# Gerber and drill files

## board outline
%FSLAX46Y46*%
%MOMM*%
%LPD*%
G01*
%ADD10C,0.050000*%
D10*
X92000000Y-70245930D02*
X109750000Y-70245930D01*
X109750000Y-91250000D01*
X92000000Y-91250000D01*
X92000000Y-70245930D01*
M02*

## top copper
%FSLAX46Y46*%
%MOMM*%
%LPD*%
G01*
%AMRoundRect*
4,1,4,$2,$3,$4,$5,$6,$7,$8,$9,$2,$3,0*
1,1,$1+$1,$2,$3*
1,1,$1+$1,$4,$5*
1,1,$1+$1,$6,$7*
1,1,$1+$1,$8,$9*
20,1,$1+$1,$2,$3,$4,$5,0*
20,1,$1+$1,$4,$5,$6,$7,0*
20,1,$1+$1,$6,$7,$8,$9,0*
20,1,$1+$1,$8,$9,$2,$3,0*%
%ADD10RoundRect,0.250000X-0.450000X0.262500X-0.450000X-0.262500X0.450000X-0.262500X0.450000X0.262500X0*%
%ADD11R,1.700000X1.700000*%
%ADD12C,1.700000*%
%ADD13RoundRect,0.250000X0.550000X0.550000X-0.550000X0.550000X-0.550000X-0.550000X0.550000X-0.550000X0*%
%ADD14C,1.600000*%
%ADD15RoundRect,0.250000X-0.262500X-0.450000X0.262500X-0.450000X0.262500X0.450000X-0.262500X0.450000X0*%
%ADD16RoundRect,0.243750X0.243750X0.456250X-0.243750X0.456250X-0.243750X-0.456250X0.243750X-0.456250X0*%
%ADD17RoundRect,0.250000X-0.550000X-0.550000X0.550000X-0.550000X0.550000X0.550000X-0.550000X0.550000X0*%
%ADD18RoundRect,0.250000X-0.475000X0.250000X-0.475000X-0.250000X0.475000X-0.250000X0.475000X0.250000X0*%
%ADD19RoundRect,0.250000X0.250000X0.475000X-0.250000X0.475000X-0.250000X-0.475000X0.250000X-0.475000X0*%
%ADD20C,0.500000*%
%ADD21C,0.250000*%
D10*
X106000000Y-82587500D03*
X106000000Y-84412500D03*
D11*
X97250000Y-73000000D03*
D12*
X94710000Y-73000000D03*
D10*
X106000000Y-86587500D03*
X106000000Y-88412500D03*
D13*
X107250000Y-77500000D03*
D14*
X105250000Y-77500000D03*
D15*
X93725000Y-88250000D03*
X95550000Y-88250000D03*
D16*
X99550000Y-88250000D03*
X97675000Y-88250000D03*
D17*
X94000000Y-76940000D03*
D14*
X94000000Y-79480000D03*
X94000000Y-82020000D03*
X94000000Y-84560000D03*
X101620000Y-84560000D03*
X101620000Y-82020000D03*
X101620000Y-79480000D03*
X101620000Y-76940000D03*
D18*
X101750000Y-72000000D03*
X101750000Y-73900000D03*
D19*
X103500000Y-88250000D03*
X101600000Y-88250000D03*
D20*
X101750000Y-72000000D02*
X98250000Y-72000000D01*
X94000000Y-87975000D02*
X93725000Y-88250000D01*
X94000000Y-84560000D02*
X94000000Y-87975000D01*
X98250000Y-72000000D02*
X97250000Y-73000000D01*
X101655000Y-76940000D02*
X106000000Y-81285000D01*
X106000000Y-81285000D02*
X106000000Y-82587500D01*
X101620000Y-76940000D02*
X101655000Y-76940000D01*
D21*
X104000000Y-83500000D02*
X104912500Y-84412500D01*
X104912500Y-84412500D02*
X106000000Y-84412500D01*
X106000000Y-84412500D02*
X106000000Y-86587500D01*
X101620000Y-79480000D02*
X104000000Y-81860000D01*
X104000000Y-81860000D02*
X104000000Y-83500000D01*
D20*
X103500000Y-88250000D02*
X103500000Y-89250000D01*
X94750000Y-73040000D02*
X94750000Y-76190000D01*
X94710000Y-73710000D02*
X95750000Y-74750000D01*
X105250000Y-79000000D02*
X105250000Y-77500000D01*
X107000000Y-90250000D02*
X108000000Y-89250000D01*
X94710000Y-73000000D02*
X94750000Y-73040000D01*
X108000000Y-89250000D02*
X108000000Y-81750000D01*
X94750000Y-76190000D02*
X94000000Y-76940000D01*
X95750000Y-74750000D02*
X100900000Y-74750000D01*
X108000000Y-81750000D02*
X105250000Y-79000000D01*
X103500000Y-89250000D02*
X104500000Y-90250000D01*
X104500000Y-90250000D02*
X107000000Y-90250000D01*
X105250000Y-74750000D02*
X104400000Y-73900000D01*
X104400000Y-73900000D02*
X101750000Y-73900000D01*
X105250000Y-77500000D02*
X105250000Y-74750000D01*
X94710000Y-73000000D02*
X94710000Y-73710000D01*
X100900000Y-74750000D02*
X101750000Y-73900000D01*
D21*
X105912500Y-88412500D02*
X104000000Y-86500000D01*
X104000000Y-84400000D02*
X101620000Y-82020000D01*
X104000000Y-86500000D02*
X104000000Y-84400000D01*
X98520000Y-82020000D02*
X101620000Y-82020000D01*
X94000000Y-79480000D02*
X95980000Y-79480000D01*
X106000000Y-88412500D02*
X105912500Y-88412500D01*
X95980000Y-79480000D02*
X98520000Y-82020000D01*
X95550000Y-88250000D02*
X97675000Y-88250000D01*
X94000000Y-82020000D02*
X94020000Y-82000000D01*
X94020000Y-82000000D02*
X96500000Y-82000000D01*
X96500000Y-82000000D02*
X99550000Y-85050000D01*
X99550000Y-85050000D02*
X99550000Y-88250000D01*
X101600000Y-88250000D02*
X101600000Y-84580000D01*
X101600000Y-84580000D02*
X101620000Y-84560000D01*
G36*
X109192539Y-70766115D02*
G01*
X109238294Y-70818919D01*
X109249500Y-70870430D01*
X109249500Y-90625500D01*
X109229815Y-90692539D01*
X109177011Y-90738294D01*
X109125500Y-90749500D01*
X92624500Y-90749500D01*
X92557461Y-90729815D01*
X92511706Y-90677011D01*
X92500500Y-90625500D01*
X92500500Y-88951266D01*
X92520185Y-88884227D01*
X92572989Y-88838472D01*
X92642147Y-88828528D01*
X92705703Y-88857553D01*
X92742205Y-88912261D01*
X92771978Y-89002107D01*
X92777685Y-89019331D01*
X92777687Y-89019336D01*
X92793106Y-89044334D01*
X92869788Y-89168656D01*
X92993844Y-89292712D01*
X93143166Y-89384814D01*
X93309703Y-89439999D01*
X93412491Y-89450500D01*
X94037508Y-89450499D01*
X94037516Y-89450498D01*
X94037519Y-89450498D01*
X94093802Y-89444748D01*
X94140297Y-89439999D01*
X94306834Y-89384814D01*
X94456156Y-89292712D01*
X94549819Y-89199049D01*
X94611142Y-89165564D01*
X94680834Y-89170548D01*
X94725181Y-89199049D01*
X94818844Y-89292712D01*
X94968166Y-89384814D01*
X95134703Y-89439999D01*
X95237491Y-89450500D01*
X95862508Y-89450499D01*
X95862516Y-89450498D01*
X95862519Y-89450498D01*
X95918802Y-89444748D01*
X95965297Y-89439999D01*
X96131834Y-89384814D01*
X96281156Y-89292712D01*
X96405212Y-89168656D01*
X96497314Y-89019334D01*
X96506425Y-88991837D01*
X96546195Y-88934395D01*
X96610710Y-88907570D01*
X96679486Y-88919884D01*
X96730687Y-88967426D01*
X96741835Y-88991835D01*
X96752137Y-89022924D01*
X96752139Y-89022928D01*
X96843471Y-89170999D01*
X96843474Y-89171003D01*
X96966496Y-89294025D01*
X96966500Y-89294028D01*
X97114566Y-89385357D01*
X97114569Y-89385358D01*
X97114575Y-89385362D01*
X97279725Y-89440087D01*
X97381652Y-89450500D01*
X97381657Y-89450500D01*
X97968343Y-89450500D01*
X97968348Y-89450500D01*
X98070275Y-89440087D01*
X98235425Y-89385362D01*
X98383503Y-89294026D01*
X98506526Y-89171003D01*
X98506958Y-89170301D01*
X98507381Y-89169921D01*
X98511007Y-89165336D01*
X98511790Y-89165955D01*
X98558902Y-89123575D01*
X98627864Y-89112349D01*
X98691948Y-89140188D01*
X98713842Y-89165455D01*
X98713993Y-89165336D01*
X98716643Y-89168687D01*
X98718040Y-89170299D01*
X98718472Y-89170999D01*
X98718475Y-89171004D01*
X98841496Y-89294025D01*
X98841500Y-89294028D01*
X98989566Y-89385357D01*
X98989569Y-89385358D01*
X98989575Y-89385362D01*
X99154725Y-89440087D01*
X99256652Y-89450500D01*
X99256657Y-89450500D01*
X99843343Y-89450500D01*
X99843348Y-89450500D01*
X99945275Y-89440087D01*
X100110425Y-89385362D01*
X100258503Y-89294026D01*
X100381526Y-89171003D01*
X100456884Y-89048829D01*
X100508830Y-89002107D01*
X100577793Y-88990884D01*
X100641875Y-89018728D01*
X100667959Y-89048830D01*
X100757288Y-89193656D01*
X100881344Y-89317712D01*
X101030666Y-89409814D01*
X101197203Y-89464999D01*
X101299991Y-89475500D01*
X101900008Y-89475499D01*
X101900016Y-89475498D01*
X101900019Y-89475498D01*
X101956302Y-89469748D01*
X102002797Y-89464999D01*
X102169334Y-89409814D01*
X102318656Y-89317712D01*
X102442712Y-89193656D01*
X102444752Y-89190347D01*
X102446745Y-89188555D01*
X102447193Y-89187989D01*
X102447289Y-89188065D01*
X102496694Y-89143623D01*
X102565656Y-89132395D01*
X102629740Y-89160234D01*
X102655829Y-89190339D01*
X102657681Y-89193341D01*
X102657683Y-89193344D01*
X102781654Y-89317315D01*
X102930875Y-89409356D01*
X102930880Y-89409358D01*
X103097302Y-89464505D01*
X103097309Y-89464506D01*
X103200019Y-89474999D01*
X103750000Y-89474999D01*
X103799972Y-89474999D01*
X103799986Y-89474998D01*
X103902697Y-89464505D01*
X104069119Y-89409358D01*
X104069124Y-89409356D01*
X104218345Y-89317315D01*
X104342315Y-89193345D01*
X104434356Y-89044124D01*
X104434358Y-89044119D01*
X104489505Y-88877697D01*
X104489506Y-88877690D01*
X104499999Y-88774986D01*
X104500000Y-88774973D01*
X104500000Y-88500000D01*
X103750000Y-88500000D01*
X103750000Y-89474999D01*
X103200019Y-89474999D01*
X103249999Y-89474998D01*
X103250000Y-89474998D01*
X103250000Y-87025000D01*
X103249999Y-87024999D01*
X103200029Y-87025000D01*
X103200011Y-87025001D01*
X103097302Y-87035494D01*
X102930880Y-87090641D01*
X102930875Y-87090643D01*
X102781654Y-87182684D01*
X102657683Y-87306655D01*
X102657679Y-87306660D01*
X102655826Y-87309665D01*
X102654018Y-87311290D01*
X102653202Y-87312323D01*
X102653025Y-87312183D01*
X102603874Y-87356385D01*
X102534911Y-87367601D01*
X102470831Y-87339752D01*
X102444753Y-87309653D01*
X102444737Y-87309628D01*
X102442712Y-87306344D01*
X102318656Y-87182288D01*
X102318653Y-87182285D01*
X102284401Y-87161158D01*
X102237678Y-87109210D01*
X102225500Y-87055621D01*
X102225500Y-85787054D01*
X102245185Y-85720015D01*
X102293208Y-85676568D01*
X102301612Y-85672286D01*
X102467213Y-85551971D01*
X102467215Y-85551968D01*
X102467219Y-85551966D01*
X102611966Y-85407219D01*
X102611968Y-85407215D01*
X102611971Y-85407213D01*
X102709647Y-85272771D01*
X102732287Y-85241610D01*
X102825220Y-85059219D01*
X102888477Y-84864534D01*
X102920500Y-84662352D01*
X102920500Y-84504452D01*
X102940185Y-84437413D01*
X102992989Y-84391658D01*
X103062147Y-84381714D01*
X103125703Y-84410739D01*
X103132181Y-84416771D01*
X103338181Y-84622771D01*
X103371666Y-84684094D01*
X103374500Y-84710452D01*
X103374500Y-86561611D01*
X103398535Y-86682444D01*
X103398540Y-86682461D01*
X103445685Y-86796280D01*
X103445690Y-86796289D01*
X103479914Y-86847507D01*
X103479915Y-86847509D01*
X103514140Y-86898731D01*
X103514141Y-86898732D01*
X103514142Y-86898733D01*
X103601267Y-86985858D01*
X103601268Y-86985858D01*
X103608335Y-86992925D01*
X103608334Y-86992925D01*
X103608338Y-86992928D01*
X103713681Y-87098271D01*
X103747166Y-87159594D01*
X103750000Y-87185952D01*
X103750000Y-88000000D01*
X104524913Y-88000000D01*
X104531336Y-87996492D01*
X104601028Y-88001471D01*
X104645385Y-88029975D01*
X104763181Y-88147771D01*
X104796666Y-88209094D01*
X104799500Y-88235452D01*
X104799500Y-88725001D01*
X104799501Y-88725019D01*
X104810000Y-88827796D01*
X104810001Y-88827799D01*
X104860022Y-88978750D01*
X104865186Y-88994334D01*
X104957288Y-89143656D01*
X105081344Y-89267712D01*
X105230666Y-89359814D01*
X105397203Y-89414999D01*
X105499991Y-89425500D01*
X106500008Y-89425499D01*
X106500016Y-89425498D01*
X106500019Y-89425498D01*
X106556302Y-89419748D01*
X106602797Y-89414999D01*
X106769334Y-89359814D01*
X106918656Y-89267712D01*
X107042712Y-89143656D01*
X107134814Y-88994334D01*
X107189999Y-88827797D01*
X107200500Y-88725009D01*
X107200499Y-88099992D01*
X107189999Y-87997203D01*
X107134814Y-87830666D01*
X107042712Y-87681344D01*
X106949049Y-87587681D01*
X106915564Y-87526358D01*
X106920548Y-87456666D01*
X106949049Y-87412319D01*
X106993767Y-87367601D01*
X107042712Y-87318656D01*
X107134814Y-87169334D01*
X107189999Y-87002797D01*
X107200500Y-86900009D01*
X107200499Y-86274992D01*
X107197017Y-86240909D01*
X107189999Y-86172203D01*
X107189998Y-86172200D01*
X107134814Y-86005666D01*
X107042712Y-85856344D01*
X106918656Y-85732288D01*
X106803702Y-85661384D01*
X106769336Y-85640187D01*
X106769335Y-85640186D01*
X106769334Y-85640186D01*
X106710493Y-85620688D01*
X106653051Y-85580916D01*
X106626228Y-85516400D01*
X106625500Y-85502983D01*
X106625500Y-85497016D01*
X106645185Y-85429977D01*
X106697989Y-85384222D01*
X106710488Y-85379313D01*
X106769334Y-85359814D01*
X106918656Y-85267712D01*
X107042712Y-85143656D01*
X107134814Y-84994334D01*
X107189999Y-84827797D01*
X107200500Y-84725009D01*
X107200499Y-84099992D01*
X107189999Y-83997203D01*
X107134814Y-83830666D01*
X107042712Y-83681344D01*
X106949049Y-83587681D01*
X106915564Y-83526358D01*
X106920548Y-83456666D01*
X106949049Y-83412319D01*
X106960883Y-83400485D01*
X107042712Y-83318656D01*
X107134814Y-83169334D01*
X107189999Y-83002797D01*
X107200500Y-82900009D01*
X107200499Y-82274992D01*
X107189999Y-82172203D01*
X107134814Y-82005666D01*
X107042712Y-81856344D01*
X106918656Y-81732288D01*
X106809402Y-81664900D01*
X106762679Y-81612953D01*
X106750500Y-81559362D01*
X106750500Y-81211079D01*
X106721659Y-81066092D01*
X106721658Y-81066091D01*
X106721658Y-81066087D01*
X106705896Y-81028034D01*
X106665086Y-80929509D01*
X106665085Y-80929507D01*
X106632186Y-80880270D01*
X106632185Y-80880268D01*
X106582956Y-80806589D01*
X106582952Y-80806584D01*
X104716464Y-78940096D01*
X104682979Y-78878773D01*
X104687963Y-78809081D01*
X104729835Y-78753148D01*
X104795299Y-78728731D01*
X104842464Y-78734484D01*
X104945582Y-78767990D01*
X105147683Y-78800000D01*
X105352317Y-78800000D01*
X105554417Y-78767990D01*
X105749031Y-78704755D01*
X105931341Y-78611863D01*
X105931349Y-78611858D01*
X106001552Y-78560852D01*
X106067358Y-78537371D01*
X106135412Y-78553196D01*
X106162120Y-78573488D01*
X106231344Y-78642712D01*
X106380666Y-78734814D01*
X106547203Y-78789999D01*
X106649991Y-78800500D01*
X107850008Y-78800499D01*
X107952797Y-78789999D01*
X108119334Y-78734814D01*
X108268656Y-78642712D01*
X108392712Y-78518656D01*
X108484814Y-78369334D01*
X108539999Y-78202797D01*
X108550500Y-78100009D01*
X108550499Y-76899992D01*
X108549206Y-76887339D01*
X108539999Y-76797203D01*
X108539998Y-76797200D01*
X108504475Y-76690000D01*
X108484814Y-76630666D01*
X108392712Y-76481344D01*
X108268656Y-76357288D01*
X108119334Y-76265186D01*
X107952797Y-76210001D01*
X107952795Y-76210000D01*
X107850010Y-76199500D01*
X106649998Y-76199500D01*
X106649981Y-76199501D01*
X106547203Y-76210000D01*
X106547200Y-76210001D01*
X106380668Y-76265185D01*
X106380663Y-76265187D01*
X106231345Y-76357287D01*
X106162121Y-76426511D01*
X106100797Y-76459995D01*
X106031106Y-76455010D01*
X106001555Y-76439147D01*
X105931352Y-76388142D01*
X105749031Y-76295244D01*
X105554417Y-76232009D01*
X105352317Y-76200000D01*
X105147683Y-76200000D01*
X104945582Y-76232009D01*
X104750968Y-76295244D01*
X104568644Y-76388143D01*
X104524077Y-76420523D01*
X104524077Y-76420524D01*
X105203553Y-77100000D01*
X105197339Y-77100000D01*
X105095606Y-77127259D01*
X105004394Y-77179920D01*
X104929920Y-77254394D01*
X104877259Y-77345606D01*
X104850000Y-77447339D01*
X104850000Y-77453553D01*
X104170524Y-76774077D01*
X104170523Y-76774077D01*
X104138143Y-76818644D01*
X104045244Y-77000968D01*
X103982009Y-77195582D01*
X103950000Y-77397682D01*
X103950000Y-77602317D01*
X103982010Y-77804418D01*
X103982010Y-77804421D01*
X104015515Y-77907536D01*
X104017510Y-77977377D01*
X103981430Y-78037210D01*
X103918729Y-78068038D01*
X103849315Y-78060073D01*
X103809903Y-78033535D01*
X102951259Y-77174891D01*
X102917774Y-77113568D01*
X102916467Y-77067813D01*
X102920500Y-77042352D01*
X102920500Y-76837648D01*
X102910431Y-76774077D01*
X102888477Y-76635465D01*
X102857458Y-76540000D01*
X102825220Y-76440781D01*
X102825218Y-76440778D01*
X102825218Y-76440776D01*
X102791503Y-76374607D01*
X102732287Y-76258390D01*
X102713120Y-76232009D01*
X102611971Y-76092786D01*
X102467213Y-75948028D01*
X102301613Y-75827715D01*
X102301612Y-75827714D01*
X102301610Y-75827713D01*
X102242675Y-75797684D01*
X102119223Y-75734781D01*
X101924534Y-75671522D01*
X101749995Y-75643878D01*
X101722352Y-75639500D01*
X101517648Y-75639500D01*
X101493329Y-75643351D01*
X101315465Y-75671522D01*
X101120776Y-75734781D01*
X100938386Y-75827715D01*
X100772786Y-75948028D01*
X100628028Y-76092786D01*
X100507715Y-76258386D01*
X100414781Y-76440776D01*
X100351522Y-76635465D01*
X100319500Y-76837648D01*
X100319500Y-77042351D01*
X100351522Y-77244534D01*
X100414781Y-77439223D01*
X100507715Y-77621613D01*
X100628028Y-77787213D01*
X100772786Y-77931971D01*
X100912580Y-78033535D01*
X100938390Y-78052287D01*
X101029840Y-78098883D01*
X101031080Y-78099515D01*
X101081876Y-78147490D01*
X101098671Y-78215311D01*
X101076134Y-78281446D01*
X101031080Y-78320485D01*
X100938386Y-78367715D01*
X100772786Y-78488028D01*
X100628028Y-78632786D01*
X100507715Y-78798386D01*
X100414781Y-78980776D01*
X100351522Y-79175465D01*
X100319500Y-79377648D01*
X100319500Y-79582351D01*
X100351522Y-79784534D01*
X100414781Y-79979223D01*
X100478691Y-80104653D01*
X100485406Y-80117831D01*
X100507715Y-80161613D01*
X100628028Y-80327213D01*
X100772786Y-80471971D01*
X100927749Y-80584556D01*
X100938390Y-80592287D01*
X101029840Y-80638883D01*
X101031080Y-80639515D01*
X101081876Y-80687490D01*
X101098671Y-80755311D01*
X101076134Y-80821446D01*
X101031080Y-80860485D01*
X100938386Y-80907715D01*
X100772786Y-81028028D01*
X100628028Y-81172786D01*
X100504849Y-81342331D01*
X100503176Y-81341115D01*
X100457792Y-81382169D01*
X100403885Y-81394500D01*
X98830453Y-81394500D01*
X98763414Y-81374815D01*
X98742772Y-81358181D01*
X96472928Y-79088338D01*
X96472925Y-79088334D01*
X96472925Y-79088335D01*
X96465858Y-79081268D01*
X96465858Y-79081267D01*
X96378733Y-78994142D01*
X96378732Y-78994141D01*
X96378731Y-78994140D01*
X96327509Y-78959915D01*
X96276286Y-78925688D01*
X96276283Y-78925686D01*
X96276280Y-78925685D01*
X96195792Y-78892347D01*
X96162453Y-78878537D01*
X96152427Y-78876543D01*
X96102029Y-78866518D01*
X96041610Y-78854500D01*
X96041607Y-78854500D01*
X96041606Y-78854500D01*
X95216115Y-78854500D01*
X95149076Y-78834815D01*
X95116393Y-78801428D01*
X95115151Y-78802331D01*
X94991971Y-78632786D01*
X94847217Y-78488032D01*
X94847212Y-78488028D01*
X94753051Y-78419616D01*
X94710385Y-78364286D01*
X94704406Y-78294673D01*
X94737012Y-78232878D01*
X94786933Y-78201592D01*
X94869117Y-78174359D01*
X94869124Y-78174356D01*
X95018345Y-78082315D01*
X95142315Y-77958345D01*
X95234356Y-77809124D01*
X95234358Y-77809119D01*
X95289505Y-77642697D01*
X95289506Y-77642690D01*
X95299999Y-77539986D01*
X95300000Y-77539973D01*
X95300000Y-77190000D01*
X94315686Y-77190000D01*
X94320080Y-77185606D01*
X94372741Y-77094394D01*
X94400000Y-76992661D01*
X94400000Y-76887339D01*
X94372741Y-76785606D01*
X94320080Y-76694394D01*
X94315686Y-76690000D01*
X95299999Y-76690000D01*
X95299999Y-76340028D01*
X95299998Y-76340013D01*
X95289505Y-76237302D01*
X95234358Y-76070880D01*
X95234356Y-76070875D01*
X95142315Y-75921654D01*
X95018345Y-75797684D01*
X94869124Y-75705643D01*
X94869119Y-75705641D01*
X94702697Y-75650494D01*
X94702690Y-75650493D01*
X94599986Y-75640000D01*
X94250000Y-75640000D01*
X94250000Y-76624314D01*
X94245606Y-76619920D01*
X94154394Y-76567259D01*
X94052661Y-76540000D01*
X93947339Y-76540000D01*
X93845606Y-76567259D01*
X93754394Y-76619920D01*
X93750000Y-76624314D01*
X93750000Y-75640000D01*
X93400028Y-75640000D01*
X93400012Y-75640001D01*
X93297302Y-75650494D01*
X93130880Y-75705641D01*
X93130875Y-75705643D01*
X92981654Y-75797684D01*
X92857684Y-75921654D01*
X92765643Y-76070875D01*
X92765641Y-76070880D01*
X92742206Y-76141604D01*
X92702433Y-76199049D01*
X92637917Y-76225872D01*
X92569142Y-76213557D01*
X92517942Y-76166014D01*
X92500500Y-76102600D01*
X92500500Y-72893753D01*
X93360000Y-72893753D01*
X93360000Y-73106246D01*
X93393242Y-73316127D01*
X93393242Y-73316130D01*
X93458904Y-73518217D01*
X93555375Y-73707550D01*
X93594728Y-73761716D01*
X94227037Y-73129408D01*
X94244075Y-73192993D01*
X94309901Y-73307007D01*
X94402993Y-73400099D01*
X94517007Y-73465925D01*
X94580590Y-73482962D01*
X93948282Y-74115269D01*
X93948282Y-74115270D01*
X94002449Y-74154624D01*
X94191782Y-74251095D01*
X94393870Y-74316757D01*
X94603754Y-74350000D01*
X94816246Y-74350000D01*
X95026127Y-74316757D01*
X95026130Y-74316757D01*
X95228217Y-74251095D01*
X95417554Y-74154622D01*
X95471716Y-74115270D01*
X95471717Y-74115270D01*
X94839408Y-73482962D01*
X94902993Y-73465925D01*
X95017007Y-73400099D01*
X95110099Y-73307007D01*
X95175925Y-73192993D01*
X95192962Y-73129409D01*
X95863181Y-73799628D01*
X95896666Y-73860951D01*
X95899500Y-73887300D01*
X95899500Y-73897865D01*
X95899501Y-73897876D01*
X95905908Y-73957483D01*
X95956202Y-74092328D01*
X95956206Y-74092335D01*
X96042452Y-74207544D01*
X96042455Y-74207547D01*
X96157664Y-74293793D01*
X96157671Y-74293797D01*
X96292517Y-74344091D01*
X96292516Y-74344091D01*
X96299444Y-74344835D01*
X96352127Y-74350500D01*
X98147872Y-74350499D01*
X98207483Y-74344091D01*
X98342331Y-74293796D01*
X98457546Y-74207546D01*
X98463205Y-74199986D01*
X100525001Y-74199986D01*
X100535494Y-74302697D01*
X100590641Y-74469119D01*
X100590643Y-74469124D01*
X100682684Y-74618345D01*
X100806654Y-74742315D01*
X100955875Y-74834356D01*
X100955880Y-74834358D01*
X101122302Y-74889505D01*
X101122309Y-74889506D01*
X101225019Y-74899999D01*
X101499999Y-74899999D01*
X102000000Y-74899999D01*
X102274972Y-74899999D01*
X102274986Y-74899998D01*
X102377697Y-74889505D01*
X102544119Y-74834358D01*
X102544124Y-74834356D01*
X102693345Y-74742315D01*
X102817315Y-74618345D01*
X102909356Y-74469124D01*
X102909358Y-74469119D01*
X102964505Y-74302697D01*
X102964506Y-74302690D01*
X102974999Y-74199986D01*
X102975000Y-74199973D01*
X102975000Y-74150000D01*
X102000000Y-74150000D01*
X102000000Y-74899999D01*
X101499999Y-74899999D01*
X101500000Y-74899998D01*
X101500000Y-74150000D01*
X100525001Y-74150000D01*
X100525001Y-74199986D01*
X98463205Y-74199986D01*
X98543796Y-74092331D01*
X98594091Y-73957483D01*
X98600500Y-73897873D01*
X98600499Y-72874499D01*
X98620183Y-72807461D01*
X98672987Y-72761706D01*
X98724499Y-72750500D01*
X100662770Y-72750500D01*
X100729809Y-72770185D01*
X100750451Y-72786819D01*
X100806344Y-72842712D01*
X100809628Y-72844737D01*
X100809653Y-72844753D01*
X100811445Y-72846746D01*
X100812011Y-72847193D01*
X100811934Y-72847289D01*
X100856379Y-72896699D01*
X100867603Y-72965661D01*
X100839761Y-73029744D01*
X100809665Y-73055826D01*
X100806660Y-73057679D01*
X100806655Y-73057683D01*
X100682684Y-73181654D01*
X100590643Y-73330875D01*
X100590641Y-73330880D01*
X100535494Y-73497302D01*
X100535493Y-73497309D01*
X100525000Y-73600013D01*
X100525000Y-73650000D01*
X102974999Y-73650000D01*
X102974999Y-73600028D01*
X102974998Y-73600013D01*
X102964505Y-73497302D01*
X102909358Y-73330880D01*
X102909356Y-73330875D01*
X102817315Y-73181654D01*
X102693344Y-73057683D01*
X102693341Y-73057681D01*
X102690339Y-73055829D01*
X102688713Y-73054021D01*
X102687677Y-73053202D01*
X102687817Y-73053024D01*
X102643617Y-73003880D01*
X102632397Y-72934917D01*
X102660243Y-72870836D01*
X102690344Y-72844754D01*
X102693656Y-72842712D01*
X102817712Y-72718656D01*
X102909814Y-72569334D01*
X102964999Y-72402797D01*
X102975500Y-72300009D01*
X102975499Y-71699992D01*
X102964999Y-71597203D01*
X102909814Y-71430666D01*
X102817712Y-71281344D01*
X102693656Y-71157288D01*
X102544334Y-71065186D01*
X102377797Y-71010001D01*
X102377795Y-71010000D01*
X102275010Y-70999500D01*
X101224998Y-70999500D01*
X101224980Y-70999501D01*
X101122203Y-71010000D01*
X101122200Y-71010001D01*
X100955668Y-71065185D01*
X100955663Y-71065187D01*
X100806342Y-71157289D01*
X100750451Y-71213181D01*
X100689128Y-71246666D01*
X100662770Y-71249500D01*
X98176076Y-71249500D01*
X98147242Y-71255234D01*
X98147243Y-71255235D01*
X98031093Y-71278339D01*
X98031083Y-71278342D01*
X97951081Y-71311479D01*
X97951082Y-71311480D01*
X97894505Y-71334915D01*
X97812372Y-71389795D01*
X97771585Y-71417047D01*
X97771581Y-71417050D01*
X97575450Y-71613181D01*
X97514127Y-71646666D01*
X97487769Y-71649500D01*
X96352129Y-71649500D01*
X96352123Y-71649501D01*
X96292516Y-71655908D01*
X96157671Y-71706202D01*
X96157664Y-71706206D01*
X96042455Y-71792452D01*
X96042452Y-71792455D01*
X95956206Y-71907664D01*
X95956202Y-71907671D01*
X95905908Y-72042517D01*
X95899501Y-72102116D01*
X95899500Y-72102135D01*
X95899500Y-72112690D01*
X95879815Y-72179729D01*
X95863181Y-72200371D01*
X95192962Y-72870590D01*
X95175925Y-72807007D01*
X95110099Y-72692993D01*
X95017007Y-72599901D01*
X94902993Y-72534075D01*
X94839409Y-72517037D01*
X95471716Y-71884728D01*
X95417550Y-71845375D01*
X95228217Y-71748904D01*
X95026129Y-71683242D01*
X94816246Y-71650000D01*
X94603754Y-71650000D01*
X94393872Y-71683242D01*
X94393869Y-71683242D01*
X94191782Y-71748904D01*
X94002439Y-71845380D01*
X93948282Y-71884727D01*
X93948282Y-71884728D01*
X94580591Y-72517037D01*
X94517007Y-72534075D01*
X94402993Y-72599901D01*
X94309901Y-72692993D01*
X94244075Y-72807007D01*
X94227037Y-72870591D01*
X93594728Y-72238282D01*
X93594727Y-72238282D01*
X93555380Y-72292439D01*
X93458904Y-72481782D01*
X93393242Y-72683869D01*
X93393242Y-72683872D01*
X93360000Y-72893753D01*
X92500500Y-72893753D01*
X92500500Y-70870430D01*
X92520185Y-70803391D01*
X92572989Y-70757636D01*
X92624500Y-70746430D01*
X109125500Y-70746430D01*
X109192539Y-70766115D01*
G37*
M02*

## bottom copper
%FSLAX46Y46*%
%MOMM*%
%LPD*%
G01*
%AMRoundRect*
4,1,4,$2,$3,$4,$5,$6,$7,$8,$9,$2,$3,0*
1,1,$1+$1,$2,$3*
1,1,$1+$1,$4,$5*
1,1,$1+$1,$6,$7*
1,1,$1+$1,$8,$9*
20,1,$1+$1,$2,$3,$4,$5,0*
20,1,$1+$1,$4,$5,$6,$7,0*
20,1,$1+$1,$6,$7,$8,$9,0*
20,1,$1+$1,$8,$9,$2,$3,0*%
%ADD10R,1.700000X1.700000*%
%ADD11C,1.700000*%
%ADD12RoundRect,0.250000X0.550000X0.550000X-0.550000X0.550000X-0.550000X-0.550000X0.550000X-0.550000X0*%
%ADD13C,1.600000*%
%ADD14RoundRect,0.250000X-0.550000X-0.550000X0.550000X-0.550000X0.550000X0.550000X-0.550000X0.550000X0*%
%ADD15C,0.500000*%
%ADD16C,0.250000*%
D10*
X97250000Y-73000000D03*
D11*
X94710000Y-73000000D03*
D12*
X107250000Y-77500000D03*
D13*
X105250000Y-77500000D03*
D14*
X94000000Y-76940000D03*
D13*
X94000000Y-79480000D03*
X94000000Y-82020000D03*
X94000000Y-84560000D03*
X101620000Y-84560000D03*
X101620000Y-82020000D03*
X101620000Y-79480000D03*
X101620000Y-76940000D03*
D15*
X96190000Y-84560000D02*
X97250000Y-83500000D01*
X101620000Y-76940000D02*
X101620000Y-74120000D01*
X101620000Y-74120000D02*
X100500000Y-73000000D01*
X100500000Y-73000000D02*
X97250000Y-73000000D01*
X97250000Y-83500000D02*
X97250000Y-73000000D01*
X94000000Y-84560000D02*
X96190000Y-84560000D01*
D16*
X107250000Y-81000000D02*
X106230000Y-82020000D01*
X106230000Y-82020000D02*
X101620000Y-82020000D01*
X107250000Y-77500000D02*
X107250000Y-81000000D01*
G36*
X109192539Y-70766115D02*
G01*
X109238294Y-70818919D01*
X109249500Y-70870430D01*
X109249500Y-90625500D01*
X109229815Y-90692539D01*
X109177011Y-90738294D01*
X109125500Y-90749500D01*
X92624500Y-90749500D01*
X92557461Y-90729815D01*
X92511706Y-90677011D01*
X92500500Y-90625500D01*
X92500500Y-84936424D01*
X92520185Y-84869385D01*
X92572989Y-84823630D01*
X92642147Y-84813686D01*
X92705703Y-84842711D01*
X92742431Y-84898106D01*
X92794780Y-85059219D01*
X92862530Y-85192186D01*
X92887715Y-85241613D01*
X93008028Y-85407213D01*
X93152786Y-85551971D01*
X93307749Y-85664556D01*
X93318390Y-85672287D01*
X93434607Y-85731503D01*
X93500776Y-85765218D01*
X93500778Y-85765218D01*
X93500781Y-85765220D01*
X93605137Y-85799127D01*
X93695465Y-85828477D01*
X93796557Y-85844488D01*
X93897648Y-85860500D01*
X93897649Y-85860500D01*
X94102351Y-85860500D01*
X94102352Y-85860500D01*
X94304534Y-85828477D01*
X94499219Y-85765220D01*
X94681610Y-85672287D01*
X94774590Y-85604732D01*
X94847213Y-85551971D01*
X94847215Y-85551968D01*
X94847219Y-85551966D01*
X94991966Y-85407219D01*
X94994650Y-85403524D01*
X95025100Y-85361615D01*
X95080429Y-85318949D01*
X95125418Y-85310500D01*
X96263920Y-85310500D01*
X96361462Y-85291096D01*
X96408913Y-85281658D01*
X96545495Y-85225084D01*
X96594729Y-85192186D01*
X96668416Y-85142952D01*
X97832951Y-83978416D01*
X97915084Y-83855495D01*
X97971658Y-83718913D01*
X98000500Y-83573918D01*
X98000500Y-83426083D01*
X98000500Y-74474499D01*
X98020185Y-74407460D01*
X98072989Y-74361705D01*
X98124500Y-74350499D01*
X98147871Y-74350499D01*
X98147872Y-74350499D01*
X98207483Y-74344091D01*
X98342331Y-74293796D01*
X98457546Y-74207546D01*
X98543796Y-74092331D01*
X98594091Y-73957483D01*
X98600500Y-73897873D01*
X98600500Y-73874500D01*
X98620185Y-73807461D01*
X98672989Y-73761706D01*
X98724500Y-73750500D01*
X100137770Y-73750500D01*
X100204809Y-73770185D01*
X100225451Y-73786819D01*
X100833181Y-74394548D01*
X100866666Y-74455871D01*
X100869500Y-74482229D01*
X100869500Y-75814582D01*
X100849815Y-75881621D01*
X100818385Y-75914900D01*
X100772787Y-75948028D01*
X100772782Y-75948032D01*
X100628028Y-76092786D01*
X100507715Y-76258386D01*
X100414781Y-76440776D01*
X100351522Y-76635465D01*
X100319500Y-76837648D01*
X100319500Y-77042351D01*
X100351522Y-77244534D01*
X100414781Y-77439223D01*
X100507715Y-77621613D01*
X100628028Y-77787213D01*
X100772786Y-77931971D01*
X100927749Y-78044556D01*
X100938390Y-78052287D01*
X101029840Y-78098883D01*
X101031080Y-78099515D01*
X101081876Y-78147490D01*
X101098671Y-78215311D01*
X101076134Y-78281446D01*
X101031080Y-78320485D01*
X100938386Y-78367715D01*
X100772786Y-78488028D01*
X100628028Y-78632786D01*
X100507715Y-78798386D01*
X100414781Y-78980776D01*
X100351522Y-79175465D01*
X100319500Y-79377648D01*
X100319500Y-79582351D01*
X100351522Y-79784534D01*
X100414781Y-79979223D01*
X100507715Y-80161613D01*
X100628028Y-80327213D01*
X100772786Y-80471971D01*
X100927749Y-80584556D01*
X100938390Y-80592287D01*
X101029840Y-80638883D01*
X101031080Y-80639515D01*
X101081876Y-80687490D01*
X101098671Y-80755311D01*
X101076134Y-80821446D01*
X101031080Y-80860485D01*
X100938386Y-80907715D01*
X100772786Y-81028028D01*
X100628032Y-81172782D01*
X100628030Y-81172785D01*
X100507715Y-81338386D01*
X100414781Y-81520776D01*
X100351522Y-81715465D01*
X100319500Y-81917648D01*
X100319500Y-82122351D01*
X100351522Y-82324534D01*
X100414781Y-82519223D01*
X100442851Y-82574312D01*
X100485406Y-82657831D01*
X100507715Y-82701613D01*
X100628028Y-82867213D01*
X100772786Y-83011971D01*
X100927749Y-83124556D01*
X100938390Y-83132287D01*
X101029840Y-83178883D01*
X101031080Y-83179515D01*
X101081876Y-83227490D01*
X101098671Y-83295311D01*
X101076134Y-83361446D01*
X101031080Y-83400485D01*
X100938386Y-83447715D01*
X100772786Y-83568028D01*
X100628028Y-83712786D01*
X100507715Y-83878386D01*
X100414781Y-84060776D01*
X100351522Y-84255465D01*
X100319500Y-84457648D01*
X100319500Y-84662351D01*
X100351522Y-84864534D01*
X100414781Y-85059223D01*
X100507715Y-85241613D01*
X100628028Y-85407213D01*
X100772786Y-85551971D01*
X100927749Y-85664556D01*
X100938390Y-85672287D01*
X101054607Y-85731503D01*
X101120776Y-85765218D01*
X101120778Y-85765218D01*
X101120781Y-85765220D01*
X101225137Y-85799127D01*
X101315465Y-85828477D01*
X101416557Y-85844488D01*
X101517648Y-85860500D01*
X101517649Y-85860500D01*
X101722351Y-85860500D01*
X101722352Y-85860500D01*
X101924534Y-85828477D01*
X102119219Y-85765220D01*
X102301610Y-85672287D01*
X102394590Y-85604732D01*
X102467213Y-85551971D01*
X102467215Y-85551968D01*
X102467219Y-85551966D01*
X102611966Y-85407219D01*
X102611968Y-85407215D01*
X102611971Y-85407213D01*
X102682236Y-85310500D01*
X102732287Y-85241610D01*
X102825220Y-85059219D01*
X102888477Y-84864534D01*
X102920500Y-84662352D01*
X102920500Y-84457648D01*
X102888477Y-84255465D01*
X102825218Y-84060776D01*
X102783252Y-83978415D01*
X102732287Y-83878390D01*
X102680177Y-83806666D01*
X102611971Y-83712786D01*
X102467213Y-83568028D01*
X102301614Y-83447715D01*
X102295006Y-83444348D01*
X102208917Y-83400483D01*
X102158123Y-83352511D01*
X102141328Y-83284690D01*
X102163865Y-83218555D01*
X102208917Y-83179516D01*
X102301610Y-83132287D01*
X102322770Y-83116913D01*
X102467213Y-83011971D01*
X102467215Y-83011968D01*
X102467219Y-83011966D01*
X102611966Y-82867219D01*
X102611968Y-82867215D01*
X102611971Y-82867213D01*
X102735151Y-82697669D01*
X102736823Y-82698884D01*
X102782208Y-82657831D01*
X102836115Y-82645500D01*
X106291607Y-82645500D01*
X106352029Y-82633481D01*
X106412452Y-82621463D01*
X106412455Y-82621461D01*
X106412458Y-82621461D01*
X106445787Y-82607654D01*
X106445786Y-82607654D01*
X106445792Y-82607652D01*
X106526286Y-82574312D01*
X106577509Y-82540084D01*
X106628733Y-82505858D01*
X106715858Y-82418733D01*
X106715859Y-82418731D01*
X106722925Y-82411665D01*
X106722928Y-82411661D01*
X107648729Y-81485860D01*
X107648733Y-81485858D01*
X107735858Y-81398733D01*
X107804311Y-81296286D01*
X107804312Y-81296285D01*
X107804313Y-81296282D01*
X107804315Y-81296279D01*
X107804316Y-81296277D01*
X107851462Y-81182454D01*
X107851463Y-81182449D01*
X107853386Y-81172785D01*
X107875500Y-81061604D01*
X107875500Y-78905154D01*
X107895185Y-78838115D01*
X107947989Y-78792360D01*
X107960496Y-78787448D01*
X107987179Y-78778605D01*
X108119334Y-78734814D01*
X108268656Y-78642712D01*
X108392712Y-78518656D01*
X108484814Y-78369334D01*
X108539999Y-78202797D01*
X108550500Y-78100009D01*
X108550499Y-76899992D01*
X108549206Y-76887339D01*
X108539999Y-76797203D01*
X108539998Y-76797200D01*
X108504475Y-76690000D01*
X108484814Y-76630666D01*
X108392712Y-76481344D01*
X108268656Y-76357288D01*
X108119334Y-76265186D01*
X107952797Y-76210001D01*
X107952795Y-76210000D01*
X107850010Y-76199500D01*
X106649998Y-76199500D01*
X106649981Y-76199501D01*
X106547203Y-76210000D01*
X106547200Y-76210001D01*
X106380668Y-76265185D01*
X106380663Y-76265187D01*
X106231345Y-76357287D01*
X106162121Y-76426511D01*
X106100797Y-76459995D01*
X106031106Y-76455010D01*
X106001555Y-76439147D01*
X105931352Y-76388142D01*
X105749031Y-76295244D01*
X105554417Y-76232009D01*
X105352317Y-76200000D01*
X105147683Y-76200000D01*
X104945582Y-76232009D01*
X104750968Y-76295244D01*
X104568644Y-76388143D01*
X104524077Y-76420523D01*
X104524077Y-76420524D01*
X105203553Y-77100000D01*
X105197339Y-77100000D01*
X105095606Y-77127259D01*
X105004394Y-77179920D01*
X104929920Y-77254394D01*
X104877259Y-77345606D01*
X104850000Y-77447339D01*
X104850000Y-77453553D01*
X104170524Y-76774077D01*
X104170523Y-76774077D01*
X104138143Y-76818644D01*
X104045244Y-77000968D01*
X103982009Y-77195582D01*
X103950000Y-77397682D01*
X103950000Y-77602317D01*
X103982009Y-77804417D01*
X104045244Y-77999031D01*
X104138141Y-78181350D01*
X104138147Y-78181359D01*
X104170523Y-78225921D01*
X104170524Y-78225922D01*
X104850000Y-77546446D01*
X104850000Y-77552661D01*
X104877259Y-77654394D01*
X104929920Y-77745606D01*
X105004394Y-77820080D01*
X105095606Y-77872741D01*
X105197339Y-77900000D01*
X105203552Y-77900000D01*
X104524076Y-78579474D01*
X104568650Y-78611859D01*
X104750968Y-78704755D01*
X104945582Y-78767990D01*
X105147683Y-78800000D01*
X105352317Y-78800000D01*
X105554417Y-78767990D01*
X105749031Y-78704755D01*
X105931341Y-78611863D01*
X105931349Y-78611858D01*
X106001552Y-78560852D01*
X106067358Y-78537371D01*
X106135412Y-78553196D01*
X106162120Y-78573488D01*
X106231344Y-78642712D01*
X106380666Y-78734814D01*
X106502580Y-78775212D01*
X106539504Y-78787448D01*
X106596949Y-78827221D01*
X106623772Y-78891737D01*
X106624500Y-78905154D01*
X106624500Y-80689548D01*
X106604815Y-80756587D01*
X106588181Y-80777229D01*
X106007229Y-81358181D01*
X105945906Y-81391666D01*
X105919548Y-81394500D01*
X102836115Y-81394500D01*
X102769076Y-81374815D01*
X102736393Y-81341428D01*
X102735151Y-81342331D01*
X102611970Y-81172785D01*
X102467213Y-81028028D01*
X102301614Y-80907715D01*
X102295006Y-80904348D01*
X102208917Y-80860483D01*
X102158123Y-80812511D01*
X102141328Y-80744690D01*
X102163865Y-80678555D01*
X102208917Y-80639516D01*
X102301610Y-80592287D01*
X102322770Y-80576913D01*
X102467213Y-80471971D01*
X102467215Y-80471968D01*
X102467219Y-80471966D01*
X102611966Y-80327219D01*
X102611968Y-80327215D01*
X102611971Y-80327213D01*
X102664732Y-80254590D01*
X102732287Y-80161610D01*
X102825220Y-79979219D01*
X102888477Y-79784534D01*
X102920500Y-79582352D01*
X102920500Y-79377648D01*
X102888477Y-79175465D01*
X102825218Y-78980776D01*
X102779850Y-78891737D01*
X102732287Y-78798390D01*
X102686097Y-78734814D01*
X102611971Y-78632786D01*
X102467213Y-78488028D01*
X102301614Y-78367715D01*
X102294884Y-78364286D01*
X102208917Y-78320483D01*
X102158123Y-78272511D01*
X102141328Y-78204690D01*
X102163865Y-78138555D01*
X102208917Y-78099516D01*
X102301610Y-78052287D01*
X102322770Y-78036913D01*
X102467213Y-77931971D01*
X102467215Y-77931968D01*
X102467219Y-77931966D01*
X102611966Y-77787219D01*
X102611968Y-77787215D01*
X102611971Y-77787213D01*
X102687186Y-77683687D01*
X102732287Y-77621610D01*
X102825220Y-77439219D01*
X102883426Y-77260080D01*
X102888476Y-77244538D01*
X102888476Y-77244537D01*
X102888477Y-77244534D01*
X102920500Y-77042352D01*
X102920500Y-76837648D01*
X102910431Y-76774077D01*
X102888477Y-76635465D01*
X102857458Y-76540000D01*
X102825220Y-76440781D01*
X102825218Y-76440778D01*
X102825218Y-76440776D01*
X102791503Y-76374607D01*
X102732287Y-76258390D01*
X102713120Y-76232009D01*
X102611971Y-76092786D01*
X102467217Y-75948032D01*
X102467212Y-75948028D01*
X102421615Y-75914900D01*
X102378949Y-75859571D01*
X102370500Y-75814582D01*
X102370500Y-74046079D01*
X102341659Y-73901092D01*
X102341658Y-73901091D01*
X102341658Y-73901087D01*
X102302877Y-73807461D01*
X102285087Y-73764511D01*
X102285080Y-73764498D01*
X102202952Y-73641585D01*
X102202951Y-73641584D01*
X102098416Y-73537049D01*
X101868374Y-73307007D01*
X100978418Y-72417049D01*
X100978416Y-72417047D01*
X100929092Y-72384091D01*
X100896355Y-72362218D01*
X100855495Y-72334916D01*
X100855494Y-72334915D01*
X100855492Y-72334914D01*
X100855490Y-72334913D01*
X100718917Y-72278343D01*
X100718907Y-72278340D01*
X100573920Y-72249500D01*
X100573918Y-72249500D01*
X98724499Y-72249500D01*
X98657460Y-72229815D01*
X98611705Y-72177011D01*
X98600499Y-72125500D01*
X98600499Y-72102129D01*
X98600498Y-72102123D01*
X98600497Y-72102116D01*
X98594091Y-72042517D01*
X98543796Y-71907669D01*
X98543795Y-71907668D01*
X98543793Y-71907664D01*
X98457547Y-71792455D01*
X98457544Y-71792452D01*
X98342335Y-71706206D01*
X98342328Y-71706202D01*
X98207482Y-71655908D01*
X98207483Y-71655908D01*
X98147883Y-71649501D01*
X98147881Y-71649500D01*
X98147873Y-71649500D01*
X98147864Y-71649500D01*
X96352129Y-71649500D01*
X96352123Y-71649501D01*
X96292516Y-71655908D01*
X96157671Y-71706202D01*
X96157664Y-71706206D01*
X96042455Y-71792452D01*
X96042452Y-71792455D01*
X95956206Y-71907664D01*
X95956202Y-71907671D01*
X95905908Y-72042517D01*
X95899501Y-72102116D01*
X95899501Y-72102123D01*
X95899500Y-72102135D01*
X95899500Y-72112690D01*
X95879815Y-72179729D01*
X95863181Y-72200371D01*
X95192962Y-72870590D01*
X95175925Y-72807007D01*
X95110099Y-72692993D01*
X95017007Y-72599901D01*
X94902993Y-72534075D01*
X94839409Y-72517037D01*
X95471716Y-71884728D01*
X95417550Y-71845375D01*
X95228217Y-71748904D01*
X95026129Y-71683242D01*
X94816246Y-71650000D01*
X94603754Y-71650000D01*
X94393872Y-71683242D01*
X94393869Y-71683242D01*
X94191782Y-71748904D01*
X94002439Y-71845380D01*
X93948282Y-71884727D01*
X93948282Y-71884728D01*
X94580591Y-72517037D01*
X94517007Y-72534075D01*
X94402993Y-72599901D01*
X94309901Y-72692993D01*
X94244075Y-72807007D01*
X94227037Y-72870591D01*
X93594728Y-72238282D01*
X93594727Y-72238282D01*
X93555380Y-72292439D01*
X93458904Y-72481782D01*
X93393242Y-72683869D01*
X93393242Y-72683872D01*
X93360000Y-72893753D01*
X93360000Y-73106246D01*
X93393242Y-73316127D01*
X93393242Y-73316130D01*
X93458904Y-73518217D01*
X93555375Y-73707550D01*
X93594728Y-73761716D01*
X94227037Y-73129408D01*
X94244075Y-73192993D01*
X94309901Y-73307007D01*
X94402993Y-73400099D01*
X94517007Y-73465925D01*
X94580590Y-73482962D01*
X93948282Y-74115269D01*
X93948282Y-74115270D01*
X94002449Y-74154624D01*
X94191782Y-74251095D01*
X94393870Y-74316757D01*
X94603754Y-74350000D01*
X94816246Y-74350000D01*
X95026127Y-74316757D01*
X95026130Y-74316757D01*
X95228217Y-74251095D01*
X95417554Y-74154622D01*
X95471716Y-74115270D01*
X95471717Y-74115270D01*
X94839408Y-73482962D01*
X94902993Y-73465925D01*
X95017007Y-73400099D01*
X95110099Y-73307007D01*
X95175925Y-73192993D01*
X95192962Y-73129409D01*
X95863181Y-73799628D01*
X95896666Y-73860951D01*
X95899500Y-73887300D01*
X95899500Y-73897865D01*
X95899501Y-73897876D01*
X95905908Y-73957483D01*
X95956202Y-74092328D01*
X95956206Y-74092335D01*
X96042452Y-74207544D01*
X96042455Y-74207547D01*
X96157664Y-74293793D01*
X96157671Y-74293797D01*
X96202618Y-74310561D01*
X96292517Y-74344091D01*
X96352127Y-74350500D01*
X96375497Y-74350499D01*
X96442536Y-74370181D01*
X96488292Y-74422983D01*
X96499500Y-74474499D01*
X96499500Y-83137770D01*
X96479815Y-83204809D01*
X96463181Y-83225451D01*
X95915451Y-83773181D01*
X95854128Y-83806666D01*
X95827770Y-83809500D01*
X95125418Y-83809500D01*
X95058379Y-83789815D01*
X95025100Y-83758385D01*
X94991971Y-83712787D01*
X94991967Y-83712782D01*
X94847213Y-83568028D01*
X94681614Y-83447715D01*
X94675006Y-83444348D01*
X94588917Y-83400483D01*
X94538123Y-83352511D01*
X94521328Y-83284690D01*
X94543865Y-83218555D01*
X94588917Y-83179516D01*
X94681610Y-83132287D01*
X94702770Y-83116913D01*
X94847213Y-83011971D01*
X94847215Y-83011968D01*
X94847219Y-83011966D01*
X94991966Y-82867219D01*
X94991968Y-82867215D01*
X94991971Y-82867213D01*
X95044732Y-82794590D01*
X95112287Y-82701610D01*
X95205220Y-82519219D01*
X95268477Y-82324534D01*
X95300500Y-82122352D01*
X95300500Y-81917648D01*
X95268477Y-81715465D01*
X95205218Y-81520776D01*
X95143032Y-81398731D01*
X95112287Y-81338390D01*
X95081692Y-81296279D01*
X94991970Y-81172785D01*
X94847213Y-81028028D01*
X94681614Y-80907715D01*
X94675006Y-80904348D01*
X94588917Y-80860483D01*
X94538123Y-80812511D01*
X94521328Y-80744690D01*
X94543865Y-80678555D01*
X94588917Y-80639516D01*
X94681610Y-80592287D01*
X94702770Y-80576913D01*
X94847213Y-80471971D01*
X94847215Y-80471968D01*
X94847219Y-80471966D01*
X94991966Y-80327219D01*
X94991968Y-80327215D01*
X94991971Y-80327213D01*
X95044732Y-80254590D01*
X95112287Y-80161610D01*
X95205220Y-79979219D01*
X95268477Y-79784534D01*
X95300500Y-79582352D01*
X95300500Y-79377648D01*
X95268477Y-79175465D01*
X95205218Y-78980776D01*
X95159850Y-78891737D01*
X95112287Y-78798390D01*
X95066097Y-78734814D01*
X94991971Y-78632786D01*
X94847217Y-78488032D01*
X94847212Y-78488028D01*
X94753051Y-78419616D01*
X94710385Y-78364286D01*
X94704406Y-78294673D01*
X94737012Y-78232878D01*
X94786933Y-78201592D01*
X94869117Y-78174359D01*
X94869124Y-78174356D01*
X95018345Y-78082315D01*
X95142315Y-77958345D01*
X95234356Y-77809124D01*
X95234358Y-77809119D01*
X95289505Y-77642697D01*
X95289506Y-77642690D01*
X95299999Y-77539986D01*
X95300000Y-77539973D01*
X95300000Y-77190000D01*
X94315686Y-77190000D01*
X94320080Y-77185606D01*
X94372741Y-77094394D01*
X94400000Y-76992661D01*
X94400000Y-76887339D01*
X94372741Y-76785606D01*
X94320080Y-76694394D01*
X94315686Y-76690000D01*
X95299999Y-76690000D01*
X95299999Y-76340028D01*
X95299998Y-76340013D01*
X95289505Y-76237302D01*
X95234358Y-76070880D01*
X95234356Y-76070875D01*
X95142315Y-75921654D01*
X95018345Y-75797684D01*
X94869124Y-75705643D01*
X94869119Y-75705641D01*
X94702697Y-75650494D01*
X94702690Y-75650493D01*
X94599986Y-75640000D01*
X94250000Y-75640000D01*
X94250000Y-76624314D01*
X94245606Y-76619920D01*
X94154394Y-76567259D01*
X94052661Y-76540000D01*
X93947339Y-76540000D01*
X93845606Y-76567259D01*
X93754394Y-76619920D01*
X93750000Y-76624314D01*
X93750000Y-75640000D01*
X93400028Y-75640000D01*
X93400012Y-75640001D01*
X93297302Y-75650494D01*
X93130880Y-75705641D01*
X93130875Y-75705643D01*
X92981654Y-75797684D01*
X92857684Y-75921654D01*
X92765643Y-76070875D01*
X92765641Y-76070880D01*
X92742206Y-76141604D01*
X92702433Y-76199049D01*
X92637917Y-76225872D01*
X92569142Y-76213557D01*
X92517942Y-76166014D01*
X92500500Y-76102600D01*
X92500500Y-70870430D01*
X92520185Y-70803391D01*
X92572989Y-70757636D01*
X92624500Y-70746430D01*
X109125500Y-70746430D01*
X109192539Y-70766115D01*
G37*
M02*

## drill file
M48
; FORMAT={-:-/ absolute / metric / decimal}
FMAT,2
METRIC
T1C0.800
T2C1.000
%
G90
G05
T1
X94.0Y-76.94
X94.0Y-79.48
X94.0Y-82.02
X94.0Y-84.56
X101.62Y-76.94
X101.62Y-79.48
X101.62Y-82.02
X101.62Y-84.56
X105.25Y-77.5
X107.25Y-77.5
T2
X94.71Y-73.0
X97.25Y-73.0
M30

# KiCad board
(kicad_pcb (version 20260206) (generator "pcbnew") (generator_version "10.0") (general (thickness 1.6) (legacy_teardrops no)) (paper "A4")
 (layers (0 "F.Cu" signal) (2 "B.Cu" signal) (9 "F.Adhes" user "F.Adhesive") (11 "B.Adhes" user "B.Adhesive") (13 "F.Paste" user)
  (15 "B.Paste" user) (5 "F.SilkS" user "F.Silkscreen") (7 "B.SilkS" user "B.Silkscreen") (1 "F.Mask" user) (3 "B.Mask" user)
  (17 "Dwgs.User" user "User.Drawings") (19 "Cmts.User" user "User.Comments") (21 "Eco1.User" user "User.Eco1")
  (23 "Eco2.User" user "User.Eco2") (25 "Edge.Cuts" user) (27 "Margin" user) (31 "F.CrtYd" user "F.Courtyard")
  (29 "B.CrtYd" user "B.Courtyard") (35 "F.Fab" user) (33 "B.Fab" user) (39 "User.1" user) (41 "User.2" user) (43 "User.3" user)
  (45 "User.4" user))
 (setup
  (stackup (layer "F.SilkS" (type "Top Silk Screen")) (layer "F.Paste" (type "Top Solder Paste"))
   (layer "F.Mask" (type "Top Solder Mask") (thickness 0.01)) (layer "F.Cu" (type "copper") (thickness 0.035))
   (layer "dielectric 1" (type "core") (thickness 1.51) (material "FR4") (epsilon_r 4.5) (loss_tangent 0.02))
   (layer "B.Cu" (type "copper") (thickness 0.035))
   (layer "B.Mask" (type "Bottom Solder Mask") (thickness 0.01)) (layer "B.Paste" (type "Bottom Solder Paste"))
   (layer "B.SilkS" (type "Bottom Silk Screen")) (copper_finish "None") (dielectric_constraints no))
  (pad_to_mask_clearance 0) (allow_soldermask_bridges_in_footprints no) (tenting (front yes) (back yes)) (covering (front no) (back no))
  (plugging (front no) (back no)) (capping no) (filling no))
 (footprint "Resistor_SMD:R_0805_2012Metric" (layer "F.Cu") (at 106 83.5 -90)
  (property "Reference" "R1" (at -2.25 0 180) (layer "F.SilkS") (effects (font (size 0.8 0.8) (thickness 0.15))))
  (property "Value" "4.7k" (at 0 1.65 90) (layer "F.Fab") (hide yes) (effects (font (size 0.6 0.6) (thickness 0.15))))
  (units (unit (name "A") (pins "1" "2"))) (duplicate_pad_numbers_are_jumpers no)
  (pad "1" smd roundrect (at -0.9125 0 270) (size 1.025 1.4) (layers "F.Cu" "F.Mask" "F.Paste") (roundrect_rratio 0.243902) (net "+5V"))
  (pad "2" smd roundrect (at 0.9125 0 270) (size 1.025 1.4) (layers "F.Cu" "F.Mask" "F.Paste") (roundrect_rratio 0.243902) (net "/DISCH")))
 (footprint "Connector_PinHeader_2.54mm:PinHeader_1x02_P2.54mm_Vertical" (layer "F.Cu") (at 97.25 73 -90)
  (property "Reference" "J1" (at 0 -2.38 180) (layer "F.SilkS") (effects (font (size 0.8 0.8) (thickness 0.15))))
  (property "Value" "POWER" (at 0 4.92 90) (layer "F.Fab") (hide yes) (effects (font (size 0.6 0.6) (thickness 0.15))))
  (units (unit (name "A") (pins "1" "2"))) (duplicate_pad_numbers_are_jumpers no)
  (pad "1" thru_hole rect (at 0 0 270) (size 1.7 1.7) (drill 1) (layers "*.Cu" "*.Mask") (remove_unused_layers no) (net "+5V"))
  (pad "2" thru_hole circle (at 0 2.54 270) (size 1.7 1.7) (drill 1) (layers "*.Cu" "*.Mask") (remove_unused_layers no) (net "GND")))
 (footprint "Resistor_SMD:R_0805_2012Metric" (layer "F.Cu") (at 106 87.5 -90)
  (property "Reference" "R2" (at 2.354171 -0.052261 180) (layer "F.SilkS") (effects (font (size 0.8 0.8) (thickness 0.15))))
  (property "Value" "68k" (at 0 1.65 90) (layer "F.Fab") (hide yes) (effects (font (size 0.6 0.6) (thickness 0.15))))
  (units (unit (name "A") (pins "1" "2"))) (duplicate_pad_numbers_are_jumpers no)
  (pad "1" smd roundrect (at -0.9125 0 270) (size 1.025 1.4) (layers "F.Cu" "F.Mask" "F.Paste") (roundrect_rratio 0.243902) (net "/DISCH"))
  (pad "2" smd roundrect (at 0.9125 0 270) (size 1.025 1.4) (layers "F.Cu" "F.Mask" "F.Paste") (roundrect_rratio 0.243902) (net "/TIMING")))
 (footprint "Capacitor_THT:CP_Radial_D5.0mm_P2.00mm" (layer "F.Cu") (at 107.25 77.5 180)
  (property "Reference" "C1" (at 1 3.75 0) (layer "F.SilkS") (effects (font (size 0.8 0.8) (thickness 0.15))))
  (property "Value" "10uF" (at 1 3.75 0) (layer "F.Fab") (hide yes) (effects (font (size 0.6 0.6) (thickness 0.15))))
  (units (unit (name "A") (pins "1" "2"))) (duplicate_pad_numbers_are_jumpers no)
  (pad "1" thru_hole roundrect (at 0 0 180) (size 1.6 1.6) (drill 0.8) (layers "*.Cu" "*.Mask") (remove_unused_layers no)
   (roundrect_rratio 0.15625) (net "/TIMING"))
  (pad "2" thru_hole circle (at 2 0 180) (size 1.6 1.6) (drill 0.8) (layers "*.Cu" "*.Mask") (remove_unused_layers no) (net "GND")))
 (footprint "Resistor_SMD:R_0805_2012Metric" (layer "F.Cu") (at 94.6375 88.25)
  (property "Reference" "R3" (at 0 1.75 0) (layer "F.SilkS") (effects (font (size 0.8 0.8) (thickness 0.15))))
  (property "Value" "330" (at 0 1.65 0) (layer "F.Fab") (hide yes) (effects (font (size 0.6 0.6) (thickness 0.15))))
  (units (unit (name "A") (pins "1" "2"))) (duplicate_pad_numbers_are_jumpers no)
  (pad "1" smd roundrect (at -0.9125 0) (size 1.025 1.4) (layers "F.Cu" "F.Mask" "F.Paste") (roundrect_rratio 0.243902) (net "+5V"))
  (pad "2" smd roundrect (at 0.9125 0) (size 1.025 1.4) (layers "F.Cu" "F.Mask" "F.Paste") (roundrect_rratio 0.243902) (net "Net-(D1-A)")))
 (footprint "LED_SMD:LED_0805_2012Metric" (layer "F.Cu") (at 98.6125 88.25 180)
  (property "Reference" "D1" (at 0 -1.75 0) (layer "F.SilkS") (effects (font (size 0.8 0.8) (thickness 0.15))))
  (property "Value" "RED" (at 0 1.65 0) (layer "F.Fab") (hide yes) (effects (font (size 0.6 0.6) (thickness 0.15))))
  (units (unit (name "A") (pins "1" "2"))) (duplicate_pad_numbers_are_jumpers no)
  (pad "1" smd roundrect (at -0.9375 0 180) (size 0.975 1.4) (layers "F.Cu" "F.Mask" "F.Paste") (roundrect_rratio 0.25) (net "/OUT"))
  (pad "2" smd roundrect (at 0.9375 0 180) (size 0.975 1.4) (layers "F.Cu" "F.Mask" "F.Paste") (roundrect_rratio 0.25) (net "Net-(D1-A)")))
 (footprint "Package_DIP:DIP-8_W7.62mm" (layer "F.Cu") (at 94 76.94)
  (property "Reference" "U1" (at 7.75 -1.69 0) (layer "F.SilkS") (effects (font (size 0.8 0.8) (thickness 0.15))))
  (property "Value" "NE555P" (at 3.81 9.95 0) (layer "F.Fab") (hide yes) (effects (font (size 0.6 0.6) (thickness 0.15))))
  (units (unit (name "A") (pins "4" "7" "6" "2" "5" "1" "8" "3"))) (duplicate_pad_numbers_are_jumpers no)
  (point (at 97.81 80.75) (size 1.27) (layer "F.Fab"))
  (pad "1" thru_hole roundrect (at 0 0) (size 1.6 1.6) (drill 0.8) (layers "*.Cu" "*.Mask") (remove_unused_layers no)
   (roundrect_rratio 0.15625) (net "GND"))
  (pad "2" thru_hole circle (at 0 2.54) (size 1.6 1.6) (drill 0.8) (layers "*.Cu" "*.Mask") (remove_unused_layers no) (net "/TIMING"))
  (pad "3" thru_hole circle (at 0 5.08) (size 1.6 1.6) (drill 0.8) (layers "*.Cu" "*.Mask") (remove_unused_layers no) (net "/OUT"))
  (pad "4" thru_hole circle (at 0 7.62) (size 1.6 1.6) (drill 0.8) (layers "*.Cu" "*.Mask") (remove_unused_layers no) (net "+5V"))
  (pad "5" thru_hole circle (at 7.62 7.62) (size 1.6 1.6) (drill 0.8) (layers "*.Cu" "*.Mask") (remove_unused_layers no) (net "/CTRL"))
  (pad "6" thru_hole circle (at 7.62 5.08) (size 1.6 1.6) (drill 0.8) (layers "*.Cu" "*.Mask") (remove_unused_layers no) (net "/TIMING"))
  (pad "7" thru_hole circle (at 7.62 2.54) (size 1.6 1.6) (drill 0.8) (layers "*.Cu" "*.Mask") (remove_unused_layers no) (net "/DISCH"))
  (pad "8" thru_hole circle (at 7.62 0) (size 1.6 1.6) (drill 0.8) (layers "*.Cu" "*.Mask") (remove_unused_layers no) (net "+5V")))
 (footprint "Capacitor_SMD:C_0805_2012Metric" (layer "F.Cu") (at 101.75 72.95 -90)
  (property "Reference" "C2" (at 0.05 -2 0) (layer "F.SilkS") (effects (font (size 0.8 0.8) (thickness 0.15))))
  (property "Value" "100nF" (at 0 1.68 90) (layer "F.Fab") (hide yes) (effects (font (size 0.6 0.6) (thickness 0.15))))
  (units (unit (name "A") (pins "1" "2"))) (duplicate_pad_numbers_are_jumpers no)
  (pad "1" smd roundrect (at -0.95 0 270) (size 1 1.45) (layers "F.Cu" "F.Mask" "F.Paste") (roundrect_rratio 0.25) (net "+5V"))
  (pad "2" smd roundrect (at 0.95 0 270) (size 1 1.45) (layers "F.Cu" "F.Mask" "F.Paste") (roundrect_rratio 0.25) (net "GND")))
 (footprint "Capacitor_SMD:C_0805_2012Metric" (layer "F.Cu") (at 102.55 88.25 180)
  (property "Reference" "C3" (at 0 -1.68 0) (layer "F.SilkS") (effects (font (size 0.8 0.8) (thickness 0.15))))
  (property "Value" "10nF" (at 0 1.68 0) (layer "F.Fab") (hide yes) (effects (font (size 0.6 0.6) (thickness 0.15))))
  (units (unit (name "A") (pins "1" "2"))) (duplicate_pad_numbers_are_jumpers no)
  (pad "1" smd roundrect (at -0.95 0 180) (size 1 1.45) (layers "F.Cu" "F.Mask" "F.Paste") (roundrect_rratio 0.25) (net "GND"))
  (pad "2" smd roundrect (at 0.95 0 180) (size 1 1.45) (layers "F.Cu" "F.Mask" "F.Paste") (roundrect_rratio 0.25) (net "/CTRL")))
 (gr_rect (start 92 70.24593) (end 109.75 91.25) (stroke (width 0.05) (type default)) (fill no) (layer "Edge.Cuts"))
 (segment (start 101.75 72) (end 98.25 72) (width 0.5) (layer "F.Cu") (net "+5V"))
 (segment (start 94 87.975) (end 93.725 88.25) (width 0.5) (layer "F.Cu") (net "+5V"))
 (segment (start 94 84.56) (end 94 87.975) (width 0.5) (layer "F.Cu") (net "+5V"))
 (segment (start 98.25 72) (end 97.25 73) (width 0.5) (layer "F.Cu") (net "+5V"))
 (segment (start 101.655 76.94) (end 106 81.285) (width 0.5) (layer "F.Cu") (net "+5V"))
 (segment (start 106 81.285) (end 106 82.5875) (width 0.5) (layer "F.Cu") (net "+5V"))
 (segment (start 101.62 76.94) (end 101.655 76.94) (width 0.5) (layer "F.Cu") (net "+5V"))
 (segment (start 96.19 84.56) (end 97.25 83.5) (width 0.5) (layer "B.Cu") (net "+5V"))
 (segment (start 101.62 76.94) (end 101.62 74.12) (width 0.5) (layer "B.Cu") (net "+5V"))
 (segment (start 101.62 74.12) (end 100.5 73) (width 0.5) (layer "B.Cu") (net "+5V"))
 (segment (start 100.5 73) (end 97.25 73) (width 0.5) (layer "B.Cu") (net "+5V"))
 (segment (start 97.25 83.5) (end 97.25 73) (width 0.5) (layer "B.Cu") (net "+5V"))
 (segment (start 94 84.56) (end 96.19 84.56) (width 0.5) (layer "B.Cu") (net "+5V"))
 (segment (start 104 83.5) (end 104.9125 84.4125) (width 0.25) (layer "F.Cu") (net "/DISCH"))
 (segment (start 104.9125 84.4125) (end 106 84.4125) (width 0.25) (layer "F.Cu") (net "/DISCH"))
 (segment (start 106 84.4125) (end 106 86.5875) (width 0.25) (layer "F.Cu") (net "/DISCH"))
 (segment (start 101.62 79.48) (end 104 81.86) (width 0.25) (layer "F.Cu") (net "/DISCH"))
 (segment (start 104 81.86) (end 104 83.5) (width 0.25) (layer "F.Cu") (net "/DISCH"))
 (segment (start 103.5 88.25) (end 103.5 89.25) (width 0.5) (layer "F.Cu") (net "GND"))
 (segment (start 94.75 73.04) (end 94.75 76.19) (width 0.5) (layer "F.Cu") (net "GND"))
 (segment (start 94.71 73.71) (end 95.75 74.75) (width 0.5) (layer "F.Cu") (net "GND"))
 (segment (start 105.25 79) (end 105.25 77.5) (width 0.5) (layer "F.Cu") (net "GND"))
 (segment (start 107 90.25) (end 108 89.25) (width 0.5) (layer "F.Cu") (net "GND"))
 (segment (start 94.71 73) (end 94.75 73.04) (width 0.5) (layer "F.Cu") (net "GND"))
 (segment (start 108 89.25) (end 108 81.75) (width 0.5) (layer "F.Cu") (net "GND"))
 (segment (start 94.75 76.19) (end 94 76.94) (width 0.5) (layer "F.Cu") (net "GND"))
 (segment (start 95.75 74.75) (end 100.9 74.75) (width 0.5) (layer "F.Cu") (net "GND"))
 (segment (start 108 81.75) (end 105.25 79) (width 0.5) (layer "F.Cu") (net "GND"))
 (segment (start 103.5 89.25) (end 104.5 90.25) (width 0.5) (layer "F.Cu") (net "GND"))
 (segment (start 104.5 90.25) (end 107 90.25) (width 0.5) (layer "F.Cu") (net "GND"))
 (segment (start 105.25 74.75) (end 104.4 73.9) (width 0.5) (layer "F.Cu") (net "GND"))
 (segment (start 104.4 73.9) (end 101.75 73.9) (width 0.5) (layer "F.Cu") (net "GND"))
 (segment (start 105.25 77.5) (end 105.25 74.75) (width 0.5) (layer "F.Cu") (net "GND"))
 (segment (start 94.71 73) (end 94.71 73.71) (width 0.5) (layer "F.Cu") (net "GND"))
 (segment (start 100.9 74.75) (end 101.75 73.9) (width 0.5) (layer "F.Cu") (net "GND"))
 (segment (start 105.9125 88.4125) (end 104 86.5) (width 0.25) (layer "F.Cu") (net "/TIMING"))
 (segment (start 104 84.4) (end 101.62 82.02) (width 0.25) (layer "F.Cu") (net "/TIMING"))
 (segment (start 104 86.5) (end 104 84.4) (width 0.25) (layer "F.Cu") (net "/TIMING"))
 (segment (start 98.52 82.02) (end 101.62 82.02) (width 0.25) (layer "F.Cu") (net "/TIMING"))
 (segment (start 94 79.48) (end 95.98 79.48) (width 0.25) (layer "F.Cu") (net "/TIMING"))
 (segment (start 106 88.4125) (end 105.9125 88.4125) (width 0.25) (layer "F.Cu") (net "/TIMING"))
 (segment (start 95.98 79.48) (end 98.52 82.02) (width 0.25) (layer "F.Cu") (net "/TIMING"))
 (segment (start 107.25 81) (end 106.23 82.02) (width 0.25) (layer "B.Cu") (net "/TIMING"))
 (segment (start 106.23 82.02) (end 101.62 82.02) (width 0.25) (layer "B.Cu") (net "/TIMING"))
 (segment (start 107.25 77.5) (end 107.25 81) (width 0.25) (layer "B.Cu") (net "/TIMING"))
 (segment (start 95.55 88.25) (end 97.675 88.25) (width 0.25) (layer "F.Cu") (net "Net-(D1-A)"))
 (segment (start 94 82.02) (end 94.02 82) (width 0.25) (layer "F.Cu") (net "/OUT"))
 (segment (start 94.02 82) (end 96.5 82) (width 0.25) (layer "F.Cu") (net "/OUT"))
 (segment (start 96.5 82) (end 99.55 85.05) (width 0.25) (layer "F.Cu") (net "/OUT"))
 (segment (start 99.55 85.05) (end 99.55 88.25) (width 0.25) (layer "F.Cu") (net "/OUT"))
 (segment (start 101.6 88.25) (end 101.6 84.58) (width 0.25) (layer "F.Cu") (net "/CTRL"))
 (segment (start 101.6 84.58) (end 101.62 84.56) (width 0.25) (layer "F.Cu") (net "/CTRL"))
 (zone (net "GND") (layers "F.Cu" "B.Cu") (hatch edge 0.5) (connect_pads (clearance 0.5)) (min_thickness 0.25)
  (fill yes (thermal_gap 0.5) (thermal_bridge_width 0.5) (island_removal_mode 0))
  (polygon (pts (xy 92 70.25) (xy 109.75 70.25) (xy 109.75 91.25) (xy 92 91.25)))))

